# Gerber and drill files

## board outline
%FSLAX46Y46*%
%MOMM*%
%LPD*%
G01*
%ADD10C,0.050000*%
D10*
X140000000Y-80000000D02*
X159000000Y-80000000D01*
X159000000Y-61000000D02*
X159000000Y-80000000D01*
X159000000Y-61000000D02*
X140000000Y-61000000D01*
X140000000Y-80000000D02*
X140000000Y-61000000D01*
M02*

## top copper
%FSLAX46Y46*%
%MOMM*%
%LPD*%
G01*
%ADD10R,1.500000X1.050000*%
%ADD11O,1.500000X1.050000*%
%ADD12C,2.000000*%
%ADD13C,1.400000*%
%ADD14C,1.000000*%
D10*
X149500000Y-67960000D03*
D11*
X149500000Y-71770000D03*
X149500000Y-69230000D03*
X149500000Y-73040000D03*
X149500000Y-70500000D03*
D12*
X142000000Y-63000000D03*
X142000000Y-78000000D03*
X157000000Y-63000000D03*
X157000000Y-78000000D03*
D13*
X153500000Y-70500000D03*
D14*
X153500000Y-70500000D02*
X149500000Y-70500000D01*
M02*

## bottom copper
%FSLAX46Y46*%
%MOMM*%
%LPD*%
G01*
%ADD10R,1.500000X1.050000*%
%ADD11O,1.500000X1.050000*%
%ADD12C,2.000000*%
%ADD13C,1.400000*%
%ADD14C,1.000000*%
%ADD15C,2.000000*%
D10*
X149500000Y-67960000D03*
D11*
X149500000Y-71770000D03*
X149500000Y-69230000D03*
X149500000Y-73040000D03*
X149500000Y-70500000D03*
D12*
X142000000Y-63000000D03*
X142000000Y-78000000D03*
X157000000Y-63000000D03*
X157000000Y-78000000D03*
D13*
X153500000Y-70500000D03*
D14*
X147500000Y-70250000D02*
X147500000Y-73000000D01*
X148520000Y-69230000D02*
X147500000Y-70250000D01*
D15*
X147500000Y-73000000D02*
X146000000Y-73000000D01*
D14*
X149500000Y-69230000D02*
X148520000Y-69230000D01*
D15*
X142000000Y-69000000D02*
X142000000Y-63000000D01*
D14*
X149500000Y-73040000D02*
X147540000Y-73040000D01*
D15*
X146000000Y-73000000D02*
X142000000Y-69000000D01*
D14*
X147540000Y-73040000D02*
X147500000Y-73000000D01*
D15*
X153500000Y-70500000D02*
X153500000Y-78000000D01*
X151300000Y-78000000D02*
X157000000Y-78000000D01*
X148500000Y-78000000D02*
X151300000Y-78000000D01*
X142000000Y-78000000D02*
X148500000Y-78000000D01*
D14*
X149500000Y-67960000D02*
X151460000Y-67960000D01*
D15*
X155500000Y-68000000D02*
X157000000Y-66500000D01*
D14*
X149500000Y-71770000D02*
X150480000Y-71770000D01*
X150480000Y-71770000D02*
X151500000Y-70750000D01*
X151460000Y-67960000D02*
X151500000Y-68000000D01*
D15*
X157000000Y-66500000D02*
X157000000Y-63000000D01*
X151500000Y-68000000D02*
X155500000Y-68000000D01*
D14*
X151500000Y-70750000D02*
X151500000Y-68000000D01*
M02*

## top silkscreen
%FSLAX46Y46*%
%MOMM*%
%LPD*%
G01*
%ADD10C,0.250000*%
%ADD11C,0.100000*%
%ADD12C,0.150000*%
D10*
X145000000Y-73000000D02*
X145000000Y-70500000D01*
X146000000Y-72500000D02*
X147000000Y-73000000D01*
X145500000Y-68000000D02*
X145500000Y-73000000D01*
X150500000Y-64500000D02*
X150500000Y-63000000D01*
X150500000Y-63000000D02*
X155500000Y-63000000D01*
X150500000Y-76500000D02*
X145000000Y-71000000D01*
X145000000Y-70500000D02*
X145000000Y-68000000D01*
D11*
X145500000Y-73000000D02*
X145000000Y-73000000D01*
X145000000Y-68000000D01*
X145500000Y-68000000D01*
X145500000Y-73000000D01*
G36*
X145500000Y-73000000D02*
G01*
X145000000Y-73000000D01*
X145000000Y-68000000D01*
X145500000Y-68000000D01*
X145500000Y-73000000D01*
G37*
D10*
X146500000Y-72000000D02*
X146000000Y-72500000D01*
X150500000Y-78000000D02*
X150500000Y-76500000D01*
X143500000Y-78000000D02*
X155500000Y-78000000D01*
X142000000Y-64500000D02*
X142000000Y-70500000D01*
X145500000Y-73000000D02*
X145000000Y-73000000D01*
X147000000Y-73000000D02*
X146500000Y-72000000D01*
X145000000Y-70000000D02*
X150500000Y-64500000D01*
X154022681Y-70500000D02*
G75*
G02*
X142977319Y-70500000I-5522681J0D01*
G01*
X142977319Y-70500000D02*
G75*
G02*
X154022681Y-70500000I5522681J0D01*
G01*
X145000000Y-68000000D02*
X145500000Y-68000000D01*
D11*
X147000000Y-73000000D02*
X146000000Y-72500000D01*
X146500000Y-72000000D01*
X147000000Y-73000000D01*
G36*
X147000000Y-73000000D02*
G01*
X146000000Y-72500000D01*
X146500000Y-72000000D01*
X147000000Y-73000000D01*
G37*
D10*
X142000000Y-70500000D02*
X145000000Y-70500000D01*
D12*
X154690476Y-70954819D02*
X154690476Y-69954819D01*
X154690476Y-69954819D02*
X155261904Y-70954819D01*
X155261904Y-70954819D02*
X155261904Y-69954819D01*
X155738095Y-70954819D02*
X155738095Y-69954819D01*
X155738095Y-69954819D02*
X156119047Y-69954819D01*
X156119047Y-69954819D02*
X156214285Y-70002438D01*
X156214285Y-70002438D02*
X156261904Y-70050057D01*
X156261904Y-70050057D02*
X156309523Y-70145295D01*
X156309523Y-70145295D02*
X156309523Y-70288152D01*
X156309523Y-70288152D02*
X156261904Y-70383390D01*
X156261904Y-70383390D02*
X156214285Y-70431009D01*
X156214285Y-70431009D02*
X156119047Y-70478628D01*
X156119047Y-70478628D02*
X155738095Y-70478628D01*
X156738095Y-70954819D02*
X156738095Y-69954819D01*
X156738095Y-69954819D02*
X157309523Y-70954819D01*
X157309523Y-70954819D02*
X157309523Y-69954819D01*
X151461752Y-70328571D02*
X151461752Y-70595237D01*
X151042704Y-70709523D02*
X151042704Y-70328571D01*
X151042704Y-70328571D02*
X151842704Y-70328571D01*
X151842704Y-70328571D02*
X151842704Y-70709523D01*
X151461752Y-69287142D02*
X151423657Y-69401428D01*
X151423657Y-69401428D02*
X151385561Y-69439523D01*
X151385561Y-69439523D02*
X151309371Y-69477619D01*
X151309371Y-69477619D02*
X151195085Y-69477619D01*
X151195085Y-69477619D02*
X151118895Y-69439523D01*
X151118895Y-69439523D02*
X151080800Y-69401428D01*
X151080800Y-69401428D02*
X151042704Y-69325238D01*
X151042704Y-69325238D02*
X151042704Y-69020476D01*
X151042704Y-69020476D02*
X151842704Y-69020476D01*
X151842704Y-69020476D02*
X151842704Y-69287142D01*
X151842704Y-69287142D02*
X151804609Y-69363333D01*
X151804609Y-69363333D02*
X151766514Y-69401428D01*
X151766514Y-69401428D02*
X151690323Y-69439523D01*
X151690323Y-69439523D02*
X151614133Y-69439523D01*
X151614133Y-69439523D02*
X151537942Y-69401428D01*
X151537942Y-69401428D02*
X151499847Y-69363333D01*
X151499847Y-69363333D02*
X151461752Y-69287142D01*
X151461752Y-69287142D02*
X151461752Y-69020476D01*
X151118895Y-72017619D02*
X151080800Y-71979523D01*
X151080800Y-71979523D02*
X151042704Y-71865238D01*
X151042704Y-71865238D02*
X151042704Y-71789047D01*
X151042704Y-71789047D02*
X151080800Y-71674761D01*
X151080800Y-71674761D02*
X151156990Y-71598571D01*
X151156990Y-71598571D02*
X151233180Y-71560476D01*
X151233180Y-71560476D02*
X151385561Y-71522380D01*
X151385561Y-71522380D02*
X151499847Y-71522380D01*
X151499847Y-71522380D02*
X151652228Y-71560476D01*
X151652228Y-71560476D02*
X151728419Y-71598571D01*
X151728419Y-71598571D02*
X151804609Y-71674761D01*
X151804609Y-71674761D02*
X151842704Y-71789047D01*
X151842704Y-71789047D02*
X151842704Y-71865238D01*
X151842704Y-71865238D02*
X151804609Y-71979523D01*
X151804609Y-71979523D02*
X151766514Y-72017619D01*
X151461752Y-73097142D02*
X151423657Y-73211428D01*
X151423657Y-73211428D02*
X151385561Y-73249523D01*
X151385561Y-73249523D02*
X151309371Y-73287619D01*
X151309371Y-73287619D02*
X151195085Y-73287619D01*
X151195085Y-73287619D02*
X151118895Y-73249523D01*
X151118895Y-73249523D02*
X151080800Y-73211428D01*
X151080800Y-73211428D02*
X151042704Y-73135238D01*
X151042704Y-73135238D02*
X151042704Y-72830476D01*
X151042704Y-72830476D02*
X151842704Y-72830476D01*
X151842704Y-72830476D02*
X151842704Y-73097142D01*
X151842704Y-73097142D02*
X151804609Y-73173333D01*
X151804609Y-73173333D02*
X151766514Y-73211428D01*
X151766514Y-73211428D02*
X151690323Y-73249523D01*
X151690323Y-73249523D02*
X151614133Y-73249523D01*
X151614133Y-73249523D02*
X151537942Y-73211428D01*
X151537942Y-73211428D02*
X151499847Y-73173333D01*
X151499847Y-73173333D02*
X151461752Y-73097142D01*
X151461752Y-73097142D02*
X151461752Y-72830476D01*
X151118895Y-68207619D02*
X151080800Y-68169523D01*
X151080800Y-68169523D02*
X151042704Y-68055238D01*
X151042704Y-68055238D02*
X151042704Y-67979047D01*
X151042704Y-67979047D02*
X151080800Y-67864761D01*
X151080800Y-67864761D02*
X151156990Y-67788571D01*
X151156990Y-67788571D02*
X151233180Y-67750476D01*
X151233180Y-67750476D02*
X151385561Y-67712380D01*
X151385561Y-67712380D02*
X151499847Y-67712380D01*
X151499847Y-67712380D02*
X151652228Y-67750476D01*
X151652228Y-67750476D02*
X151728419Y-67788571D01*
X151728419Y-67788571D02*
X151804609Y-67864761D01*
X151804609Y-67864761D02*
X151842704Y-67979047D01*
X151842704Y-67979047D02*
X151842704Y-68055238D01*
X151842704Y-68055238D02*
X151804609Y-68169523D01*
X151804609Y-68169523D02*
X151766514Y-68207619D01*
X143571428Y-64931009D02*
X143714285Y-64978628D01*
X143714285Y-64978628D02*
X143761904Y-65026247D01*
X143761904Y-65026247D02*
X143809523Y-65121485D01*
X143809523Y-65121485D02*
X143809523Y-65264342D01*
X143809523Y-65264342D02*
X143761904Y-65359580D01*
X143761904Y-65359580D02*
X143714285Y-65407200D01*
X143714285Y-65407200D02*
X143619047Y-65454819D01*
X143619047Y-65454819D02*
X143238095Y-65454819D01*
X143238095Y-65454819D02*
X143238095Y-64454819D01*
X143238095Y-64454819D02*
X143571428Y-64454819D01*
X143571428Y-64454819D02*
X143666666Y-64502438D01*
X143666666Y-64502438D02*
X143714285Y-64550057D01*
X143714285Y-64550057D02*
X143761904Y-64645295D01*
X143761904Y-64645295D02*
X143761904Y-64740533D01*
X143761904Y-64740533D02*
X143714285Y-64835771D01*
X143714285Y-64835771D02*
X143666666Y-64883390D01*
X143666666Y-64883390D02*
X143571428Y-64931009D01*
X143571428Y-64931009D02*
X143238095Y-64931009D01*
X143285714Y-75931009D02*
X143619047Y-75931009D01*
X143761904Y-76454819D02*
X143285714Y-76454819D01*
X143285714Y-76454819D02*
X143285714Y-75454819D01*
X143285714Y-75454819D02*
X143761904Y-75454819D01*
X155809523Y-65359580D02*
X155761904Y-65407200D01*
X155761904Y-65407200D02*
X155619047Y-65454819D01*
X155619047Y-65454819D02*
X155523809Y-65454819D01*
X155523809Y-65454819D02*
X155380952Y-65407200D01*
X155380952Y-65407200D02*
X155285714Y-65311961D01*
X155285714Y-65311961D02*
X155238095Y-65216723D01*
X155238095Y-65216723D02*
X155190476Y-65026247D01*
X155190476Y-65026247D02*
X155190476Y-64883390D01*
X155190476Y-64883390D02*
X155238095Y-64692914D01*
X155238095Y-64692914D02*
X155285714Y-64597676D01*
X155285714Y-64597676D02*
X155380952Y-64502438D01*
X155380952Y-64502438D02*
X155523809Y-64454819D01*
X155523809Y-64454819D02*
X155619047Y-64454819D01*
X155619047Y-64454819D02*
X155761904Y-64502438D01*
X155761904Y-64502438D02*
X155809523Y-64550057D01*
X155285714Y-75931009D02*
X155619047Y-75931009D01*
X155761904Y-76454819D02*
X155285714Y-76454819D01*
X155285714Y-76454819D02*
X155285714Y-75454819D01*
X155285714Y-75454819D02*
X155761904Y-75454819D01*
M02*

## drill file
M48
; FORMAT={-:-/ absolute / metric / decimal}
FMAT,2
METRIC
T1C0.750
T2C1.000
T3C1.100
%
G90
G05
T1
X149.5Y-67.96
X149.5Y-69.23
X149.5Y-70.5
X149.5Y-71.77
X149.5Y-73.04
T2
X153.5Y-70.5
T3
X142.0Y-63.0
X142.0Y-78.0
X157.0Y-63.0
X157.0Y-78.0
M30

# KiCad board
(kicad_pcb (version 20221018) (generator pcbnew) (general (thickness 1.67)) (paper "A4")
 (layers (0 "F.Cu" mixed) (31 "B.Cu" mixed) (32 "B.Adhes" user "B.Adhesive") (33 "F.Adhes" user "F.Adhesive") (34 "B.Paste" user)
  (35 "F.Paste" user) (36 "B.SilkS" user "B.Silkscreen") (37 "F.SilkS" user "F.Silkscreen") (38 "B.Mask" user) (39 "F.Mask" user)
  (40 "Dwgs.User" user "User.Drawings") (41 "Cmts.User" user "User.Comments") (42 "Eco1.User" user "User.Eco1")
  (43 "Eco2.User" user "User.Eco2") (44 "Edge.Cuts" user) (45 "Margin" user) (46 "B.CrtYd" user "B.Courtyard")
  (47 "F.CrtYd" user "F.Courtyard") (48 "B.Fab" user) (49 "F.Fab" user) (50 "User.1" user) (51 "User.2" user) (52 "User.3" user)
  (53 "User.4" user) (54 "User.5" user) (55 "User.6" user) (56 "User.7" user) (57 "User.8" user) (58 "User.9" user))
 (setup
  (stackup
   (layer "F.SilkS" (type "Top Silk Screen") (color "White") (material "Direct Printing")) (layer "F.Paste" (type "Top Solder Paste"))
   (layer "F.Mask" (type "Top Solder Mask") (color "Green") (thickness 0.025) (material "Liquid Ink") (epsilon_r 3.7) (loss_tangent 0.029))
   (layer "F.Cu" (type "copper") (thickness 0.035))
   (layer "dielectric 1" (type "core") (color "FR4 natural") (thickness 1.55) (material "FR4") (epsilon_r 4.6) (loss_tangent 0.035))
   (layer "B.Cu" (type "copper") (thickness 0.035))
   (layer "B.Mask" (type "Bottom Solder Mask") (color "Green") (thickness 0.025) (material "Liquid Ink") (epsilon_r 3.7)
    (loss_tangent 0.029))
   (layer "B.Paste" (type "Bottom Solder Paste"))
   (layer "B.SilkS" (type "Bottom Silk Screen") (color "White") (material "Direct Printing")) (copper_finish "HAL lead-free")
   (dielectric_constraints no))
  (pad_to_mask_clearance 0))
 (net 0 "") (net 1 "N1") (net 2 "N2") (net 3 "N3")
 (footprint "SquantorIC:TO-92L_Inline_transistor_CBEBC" (layer "F.Cu") (at 149.5 70.5 -90)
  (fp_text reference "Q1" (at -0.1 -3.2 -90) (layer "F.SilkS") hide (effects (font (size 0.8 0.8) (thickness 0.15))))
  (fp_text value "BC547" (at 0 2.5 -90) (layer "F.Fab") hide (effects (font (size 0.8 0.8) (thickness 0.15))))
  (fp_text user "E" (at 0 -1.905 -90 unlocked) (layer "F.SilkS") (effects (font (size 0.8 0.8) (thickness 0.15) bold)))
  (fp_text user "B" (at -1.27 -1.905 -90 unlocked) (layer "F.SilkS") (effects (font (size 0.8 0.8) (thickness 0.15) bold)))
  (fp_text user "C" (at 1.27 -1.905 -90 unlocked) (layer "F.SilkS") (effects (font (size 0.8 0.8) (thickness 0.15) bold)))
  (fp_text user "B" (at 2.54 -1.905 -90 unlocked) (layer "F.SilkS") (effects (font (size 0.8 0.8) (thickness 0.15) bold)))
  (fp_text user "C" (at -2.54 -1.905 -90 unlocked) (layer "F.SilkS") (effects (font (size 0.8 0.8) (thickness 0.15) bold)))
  (pad "1" thru_hole rect (at -2.54 0 270) (size 1.05 1.5) (drill 0.75) (layers "*.Cu" "*.Mask") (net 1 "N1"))
  (pad "1" thru_hole oval (at 1.27 0 270) (size 1.05 1.5) (drill 0.75) (layers "*.Cu" "*.Mask") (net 1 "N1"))
  (pad "2" thru_hole oval (at -1.27 0 270) (size 1.05 1.5) (drill 0.75) (layers "*.Cu" "*.Mask") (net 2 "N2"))
  (pad "2" thru_hole oval (at 2.54 0 270) (size 1.05 1.5) (drill 0.75) (layers "*.Cu" "*.Mask") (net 2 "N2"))
  (pad "3" thru_hole oval (at 0 0 270) (size 1.05 1.5) (drill 0.75) (layers "*.Cu" "*.Mask") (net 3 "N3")))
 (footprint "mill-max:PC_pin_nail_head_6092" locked (layer "F.Cu") (at 142 63)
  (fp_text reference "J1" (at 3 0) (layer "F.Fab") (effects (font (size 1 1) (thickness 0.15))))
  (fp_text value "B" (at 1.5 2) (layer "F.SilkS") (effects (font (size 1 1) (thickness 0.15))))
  (pad "1" thru_hole circle locked (at 0 0) (size 2 2) (drill 1.1) (layers "*.Cu" "*.Mask") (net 2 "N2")))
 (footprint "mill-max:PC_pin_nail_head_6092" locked (layer "F.Cu") (at 142 78)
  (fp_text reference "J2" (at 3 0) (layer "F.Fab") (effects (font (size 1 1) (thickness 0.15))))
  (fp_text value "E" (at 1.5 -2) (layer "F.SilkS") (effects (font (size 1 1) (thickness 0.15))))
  (pad "1" thru_hole circle locked (at 0 0) (size 2 2) (drill 1.1) (layers "*.Cu" "*.Mask") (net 3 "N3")))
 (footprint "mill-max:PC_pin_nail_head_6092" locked (layer "F.Cu") (at 157 63)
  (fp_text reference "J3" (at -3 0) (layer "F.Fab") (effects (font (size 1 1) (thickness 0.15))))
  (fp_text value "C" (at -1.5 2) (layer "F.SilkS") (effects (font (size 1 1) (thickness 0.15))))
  (pad "1" thru_hole circle locked (at 0 0) (size 2 2) (drill 1.1) (layers "*.Cu" "*.Mask") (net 1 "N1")))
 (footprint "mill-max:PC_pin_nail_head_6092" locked (layer "F.Cu") (at 157 78)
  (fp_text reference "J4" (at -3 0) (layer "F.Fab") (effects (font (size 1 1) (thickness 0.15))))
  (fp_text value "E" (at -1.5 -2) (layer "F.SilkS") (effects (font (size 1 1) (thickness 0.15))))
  (pad "1" thru_hole circle locked (at 0 0) (size 2 2) (drill 1.1) (layers "*.Cu" "*.Mask") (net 3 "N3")))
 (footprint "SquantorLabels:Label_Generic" (layer "B.Cu") (at 157.25 70.75 90)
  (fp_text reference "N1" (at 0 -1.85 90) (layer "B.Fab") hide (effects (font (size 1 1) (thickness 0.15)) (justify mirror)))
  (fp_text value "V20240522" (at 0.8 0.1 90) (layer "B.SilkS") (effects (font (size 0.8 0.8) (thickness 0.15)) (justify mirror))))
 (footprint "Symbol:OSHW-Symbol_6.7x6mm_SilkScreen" (layer "B.Cu") (at 153.75 70.5 -90)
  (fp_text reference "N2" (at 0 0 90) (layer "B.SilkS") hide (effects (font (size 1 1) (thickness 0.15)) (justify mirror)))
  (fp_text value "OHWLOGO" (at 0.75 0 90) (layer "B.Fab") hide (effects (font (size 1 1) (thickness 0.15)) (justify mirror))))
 (gr_line (start 145 73) (end 145 70.5) (stroke (width 0.25) (type solid)) (layer "F.SilkS"))
 (gr_line (start 146 72.5) (end 147 73) (stroke (width 0.25) (type solid)) (layer "F.SilkS"))
 (gr_line (start 145.5 68) (end 145.5 73) (stroke (width 0.25) (type solid)) (layer "F.SilkS"))
 (gr_line (start 150.5 64.5) (end 150.5 63) (stroke (width 0.25) (type solid)) (layer "F.SilkS"))
 (gr_line (start 150.5 63) (end 155.5 63) (stroke (width 0.25) (type solid)) (layer "F.SilkS"))
 (gr_line (start 150.5 76.5) (end 145 71) (stroke (width 0.25) (type solid)) (layer "F.SilkS"))
 (gr_line (start 145 70.5) (end 145 68) (stroke (width 0.25) (type solid)) (layer "F.SilkS"))
 (gr_poly (pts (xy 145.5 73) (xy 145 73) (xy 145 68) (xy 145.5 68)) (stroke (width 0.1) (type solid)) (fill solid) (layer "F.SilkS"))
 (gr_line (start 146.5 72) (end 146 72.5) (stroke (width 0.25) (type solid)) (layer "F.SilkS"))
 (gr_line (start 150.5 78) (end 150.5 76.5) (stroke (width 0.25) (type solid)) (layer "F.SilkS"))
 (gr_line (start 143.5 78) (end 155.5 78) (stroke (width 0.25) (type solid)) (layer "F.SilkS"))
 (gr_line (start 142 64.5) (end 142 70.5) (stroke (width 0.25) (type solid)) (layer "F.SilkS"))
 (gr_line (start 145.5 73) (end 145 73) (stroke (width 0.25) (type solid)) (layer "F.SilkS"))
 (gr_line (start 147 73) (end 146.5 72) (stroke (width 0.25) (type solid)) (layer "F.SilkS"))
 (gr_line (start 145 70) (end 150.5 64.5) (stroke (width 0.25) (type solid)) (layer "F.SilkS"))
 (gr_circle (center 148.5 70.5) (end 154 71) (stroke (width 0.25) (type solid)) (fill none) (layer "F.SilkS"))
 (gr_line (start 145 68) (end 145.5 68) (stroke (width 0.25) (type solid)) (layer "F.SilkS"))
 (gr_poly (pts (xy 147 73) (xy 146 72.5) (xy 146.5 72)) (stroke (width 0.1) (type solid)) (fill solid) (layer "F.SilkS"))
 (gr_line (start 142 70.5) (end 145 70.5) (stroke (width 0.25) (type solid)) (layer "F.SilkS"))
 (gr_line (start 140 80) (end 159 80) (stroke (width 0.05) (type solid)) (layer "Edge.Cuts"))
 (gr_line (start 159 61) (end 159 80) (stroke (width 0.05) (type solid)) (layer "Edge.Cuts"))
 (gr_line (start 159 61) (end 140 61) (stroke (width 0.05) (type solid)) (layer "Edge.Cuts"))
 (gr_line (start 140 80) (end 140 61) (stroke (width 0.05) (type solid)) (layer "Edge.Cuts"))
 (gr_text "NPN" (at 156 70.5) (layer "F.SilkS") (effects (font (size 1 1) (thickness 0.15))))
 (segment (start 147.5 70.25) (end 147.5 73) (width 1) (layer "B.Cu") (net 2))
 (segment (start 148.52 69.23) (end 147.5 70.25) (width 1) (layer "B.Cu") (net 2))
 (segment (start 147.5 73) (end 146 73) (width 2) (layer "B.Cu") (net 2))
 (segment (start 149.5 69.23) (end 148.52 69.23) (width 1) (layer "B.Cu") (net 2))
 (segment (start 142 69) (end 142 63) (width 2) (layer "B.Cu") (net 2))
 (segment (start 149.5 73.04) (end 147.54 73.04) (width 1) (layer "B.Cu") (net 2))
 (segment (start 146 73) (end 142 69) (width 2) (layer "B.Cu") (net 2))
 (segment (start 147.54 73.04) (end 147.5 73) (width 1) (layer "B.Cu") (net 2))
 (segment (start 153.5 70.5) (end 149.5 70.5) (width 1) (layer "F.Cu") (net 3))
 (via (at 153.5 70.5) (size 1.4) (drill 1) (layers "F.Cu" "B.Cu") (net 3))
 (segment (start 153.5 70.5) (end 153.5 78) (width 2) (layer "B.Cu") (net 3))
 (segment (start 151.3 78) (end 157 78) (width 2) (layer "B.Cu") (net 3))
 (segment (start 148.5 78) (end 151.3 78) (width 2) (layer "B.Cu") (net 3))
 (segment (start 142 78) (end 148.5 78) (width 2) (layer "B.Cu") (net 3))
 (segment (start 149.5 67.96) (end 151.46 67.96) (width 1) (layer "B.Cu") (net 1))
 (segment (start 155.5 68) (end 157 66.5) (width 2) (layer "B.Cu") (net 1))
 (segment (start 149.5 71.77) (end 150.48 71.77) (width 1) (layer "B.Cu") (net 1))
 (segment (start 150.48 71.77) (end 151.5 70.75) (width 1) (layer "B.Cu") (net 1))
 (segment (start 151.46 67.96) (end 151.5 68) (width 1) (layer "B.Cu") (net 1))
 (segment (start 157 66.5) (end 157 63) (width 2) (layer "B.Cu") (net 1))
 (segment (start 151.5 68) (end 155.5 68) (width 2) (layer "B.Cu") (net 1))
 (segment (start 151.5 70.75) (end 151.5 68) (width 1) (layer "B.Cu") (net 1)))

